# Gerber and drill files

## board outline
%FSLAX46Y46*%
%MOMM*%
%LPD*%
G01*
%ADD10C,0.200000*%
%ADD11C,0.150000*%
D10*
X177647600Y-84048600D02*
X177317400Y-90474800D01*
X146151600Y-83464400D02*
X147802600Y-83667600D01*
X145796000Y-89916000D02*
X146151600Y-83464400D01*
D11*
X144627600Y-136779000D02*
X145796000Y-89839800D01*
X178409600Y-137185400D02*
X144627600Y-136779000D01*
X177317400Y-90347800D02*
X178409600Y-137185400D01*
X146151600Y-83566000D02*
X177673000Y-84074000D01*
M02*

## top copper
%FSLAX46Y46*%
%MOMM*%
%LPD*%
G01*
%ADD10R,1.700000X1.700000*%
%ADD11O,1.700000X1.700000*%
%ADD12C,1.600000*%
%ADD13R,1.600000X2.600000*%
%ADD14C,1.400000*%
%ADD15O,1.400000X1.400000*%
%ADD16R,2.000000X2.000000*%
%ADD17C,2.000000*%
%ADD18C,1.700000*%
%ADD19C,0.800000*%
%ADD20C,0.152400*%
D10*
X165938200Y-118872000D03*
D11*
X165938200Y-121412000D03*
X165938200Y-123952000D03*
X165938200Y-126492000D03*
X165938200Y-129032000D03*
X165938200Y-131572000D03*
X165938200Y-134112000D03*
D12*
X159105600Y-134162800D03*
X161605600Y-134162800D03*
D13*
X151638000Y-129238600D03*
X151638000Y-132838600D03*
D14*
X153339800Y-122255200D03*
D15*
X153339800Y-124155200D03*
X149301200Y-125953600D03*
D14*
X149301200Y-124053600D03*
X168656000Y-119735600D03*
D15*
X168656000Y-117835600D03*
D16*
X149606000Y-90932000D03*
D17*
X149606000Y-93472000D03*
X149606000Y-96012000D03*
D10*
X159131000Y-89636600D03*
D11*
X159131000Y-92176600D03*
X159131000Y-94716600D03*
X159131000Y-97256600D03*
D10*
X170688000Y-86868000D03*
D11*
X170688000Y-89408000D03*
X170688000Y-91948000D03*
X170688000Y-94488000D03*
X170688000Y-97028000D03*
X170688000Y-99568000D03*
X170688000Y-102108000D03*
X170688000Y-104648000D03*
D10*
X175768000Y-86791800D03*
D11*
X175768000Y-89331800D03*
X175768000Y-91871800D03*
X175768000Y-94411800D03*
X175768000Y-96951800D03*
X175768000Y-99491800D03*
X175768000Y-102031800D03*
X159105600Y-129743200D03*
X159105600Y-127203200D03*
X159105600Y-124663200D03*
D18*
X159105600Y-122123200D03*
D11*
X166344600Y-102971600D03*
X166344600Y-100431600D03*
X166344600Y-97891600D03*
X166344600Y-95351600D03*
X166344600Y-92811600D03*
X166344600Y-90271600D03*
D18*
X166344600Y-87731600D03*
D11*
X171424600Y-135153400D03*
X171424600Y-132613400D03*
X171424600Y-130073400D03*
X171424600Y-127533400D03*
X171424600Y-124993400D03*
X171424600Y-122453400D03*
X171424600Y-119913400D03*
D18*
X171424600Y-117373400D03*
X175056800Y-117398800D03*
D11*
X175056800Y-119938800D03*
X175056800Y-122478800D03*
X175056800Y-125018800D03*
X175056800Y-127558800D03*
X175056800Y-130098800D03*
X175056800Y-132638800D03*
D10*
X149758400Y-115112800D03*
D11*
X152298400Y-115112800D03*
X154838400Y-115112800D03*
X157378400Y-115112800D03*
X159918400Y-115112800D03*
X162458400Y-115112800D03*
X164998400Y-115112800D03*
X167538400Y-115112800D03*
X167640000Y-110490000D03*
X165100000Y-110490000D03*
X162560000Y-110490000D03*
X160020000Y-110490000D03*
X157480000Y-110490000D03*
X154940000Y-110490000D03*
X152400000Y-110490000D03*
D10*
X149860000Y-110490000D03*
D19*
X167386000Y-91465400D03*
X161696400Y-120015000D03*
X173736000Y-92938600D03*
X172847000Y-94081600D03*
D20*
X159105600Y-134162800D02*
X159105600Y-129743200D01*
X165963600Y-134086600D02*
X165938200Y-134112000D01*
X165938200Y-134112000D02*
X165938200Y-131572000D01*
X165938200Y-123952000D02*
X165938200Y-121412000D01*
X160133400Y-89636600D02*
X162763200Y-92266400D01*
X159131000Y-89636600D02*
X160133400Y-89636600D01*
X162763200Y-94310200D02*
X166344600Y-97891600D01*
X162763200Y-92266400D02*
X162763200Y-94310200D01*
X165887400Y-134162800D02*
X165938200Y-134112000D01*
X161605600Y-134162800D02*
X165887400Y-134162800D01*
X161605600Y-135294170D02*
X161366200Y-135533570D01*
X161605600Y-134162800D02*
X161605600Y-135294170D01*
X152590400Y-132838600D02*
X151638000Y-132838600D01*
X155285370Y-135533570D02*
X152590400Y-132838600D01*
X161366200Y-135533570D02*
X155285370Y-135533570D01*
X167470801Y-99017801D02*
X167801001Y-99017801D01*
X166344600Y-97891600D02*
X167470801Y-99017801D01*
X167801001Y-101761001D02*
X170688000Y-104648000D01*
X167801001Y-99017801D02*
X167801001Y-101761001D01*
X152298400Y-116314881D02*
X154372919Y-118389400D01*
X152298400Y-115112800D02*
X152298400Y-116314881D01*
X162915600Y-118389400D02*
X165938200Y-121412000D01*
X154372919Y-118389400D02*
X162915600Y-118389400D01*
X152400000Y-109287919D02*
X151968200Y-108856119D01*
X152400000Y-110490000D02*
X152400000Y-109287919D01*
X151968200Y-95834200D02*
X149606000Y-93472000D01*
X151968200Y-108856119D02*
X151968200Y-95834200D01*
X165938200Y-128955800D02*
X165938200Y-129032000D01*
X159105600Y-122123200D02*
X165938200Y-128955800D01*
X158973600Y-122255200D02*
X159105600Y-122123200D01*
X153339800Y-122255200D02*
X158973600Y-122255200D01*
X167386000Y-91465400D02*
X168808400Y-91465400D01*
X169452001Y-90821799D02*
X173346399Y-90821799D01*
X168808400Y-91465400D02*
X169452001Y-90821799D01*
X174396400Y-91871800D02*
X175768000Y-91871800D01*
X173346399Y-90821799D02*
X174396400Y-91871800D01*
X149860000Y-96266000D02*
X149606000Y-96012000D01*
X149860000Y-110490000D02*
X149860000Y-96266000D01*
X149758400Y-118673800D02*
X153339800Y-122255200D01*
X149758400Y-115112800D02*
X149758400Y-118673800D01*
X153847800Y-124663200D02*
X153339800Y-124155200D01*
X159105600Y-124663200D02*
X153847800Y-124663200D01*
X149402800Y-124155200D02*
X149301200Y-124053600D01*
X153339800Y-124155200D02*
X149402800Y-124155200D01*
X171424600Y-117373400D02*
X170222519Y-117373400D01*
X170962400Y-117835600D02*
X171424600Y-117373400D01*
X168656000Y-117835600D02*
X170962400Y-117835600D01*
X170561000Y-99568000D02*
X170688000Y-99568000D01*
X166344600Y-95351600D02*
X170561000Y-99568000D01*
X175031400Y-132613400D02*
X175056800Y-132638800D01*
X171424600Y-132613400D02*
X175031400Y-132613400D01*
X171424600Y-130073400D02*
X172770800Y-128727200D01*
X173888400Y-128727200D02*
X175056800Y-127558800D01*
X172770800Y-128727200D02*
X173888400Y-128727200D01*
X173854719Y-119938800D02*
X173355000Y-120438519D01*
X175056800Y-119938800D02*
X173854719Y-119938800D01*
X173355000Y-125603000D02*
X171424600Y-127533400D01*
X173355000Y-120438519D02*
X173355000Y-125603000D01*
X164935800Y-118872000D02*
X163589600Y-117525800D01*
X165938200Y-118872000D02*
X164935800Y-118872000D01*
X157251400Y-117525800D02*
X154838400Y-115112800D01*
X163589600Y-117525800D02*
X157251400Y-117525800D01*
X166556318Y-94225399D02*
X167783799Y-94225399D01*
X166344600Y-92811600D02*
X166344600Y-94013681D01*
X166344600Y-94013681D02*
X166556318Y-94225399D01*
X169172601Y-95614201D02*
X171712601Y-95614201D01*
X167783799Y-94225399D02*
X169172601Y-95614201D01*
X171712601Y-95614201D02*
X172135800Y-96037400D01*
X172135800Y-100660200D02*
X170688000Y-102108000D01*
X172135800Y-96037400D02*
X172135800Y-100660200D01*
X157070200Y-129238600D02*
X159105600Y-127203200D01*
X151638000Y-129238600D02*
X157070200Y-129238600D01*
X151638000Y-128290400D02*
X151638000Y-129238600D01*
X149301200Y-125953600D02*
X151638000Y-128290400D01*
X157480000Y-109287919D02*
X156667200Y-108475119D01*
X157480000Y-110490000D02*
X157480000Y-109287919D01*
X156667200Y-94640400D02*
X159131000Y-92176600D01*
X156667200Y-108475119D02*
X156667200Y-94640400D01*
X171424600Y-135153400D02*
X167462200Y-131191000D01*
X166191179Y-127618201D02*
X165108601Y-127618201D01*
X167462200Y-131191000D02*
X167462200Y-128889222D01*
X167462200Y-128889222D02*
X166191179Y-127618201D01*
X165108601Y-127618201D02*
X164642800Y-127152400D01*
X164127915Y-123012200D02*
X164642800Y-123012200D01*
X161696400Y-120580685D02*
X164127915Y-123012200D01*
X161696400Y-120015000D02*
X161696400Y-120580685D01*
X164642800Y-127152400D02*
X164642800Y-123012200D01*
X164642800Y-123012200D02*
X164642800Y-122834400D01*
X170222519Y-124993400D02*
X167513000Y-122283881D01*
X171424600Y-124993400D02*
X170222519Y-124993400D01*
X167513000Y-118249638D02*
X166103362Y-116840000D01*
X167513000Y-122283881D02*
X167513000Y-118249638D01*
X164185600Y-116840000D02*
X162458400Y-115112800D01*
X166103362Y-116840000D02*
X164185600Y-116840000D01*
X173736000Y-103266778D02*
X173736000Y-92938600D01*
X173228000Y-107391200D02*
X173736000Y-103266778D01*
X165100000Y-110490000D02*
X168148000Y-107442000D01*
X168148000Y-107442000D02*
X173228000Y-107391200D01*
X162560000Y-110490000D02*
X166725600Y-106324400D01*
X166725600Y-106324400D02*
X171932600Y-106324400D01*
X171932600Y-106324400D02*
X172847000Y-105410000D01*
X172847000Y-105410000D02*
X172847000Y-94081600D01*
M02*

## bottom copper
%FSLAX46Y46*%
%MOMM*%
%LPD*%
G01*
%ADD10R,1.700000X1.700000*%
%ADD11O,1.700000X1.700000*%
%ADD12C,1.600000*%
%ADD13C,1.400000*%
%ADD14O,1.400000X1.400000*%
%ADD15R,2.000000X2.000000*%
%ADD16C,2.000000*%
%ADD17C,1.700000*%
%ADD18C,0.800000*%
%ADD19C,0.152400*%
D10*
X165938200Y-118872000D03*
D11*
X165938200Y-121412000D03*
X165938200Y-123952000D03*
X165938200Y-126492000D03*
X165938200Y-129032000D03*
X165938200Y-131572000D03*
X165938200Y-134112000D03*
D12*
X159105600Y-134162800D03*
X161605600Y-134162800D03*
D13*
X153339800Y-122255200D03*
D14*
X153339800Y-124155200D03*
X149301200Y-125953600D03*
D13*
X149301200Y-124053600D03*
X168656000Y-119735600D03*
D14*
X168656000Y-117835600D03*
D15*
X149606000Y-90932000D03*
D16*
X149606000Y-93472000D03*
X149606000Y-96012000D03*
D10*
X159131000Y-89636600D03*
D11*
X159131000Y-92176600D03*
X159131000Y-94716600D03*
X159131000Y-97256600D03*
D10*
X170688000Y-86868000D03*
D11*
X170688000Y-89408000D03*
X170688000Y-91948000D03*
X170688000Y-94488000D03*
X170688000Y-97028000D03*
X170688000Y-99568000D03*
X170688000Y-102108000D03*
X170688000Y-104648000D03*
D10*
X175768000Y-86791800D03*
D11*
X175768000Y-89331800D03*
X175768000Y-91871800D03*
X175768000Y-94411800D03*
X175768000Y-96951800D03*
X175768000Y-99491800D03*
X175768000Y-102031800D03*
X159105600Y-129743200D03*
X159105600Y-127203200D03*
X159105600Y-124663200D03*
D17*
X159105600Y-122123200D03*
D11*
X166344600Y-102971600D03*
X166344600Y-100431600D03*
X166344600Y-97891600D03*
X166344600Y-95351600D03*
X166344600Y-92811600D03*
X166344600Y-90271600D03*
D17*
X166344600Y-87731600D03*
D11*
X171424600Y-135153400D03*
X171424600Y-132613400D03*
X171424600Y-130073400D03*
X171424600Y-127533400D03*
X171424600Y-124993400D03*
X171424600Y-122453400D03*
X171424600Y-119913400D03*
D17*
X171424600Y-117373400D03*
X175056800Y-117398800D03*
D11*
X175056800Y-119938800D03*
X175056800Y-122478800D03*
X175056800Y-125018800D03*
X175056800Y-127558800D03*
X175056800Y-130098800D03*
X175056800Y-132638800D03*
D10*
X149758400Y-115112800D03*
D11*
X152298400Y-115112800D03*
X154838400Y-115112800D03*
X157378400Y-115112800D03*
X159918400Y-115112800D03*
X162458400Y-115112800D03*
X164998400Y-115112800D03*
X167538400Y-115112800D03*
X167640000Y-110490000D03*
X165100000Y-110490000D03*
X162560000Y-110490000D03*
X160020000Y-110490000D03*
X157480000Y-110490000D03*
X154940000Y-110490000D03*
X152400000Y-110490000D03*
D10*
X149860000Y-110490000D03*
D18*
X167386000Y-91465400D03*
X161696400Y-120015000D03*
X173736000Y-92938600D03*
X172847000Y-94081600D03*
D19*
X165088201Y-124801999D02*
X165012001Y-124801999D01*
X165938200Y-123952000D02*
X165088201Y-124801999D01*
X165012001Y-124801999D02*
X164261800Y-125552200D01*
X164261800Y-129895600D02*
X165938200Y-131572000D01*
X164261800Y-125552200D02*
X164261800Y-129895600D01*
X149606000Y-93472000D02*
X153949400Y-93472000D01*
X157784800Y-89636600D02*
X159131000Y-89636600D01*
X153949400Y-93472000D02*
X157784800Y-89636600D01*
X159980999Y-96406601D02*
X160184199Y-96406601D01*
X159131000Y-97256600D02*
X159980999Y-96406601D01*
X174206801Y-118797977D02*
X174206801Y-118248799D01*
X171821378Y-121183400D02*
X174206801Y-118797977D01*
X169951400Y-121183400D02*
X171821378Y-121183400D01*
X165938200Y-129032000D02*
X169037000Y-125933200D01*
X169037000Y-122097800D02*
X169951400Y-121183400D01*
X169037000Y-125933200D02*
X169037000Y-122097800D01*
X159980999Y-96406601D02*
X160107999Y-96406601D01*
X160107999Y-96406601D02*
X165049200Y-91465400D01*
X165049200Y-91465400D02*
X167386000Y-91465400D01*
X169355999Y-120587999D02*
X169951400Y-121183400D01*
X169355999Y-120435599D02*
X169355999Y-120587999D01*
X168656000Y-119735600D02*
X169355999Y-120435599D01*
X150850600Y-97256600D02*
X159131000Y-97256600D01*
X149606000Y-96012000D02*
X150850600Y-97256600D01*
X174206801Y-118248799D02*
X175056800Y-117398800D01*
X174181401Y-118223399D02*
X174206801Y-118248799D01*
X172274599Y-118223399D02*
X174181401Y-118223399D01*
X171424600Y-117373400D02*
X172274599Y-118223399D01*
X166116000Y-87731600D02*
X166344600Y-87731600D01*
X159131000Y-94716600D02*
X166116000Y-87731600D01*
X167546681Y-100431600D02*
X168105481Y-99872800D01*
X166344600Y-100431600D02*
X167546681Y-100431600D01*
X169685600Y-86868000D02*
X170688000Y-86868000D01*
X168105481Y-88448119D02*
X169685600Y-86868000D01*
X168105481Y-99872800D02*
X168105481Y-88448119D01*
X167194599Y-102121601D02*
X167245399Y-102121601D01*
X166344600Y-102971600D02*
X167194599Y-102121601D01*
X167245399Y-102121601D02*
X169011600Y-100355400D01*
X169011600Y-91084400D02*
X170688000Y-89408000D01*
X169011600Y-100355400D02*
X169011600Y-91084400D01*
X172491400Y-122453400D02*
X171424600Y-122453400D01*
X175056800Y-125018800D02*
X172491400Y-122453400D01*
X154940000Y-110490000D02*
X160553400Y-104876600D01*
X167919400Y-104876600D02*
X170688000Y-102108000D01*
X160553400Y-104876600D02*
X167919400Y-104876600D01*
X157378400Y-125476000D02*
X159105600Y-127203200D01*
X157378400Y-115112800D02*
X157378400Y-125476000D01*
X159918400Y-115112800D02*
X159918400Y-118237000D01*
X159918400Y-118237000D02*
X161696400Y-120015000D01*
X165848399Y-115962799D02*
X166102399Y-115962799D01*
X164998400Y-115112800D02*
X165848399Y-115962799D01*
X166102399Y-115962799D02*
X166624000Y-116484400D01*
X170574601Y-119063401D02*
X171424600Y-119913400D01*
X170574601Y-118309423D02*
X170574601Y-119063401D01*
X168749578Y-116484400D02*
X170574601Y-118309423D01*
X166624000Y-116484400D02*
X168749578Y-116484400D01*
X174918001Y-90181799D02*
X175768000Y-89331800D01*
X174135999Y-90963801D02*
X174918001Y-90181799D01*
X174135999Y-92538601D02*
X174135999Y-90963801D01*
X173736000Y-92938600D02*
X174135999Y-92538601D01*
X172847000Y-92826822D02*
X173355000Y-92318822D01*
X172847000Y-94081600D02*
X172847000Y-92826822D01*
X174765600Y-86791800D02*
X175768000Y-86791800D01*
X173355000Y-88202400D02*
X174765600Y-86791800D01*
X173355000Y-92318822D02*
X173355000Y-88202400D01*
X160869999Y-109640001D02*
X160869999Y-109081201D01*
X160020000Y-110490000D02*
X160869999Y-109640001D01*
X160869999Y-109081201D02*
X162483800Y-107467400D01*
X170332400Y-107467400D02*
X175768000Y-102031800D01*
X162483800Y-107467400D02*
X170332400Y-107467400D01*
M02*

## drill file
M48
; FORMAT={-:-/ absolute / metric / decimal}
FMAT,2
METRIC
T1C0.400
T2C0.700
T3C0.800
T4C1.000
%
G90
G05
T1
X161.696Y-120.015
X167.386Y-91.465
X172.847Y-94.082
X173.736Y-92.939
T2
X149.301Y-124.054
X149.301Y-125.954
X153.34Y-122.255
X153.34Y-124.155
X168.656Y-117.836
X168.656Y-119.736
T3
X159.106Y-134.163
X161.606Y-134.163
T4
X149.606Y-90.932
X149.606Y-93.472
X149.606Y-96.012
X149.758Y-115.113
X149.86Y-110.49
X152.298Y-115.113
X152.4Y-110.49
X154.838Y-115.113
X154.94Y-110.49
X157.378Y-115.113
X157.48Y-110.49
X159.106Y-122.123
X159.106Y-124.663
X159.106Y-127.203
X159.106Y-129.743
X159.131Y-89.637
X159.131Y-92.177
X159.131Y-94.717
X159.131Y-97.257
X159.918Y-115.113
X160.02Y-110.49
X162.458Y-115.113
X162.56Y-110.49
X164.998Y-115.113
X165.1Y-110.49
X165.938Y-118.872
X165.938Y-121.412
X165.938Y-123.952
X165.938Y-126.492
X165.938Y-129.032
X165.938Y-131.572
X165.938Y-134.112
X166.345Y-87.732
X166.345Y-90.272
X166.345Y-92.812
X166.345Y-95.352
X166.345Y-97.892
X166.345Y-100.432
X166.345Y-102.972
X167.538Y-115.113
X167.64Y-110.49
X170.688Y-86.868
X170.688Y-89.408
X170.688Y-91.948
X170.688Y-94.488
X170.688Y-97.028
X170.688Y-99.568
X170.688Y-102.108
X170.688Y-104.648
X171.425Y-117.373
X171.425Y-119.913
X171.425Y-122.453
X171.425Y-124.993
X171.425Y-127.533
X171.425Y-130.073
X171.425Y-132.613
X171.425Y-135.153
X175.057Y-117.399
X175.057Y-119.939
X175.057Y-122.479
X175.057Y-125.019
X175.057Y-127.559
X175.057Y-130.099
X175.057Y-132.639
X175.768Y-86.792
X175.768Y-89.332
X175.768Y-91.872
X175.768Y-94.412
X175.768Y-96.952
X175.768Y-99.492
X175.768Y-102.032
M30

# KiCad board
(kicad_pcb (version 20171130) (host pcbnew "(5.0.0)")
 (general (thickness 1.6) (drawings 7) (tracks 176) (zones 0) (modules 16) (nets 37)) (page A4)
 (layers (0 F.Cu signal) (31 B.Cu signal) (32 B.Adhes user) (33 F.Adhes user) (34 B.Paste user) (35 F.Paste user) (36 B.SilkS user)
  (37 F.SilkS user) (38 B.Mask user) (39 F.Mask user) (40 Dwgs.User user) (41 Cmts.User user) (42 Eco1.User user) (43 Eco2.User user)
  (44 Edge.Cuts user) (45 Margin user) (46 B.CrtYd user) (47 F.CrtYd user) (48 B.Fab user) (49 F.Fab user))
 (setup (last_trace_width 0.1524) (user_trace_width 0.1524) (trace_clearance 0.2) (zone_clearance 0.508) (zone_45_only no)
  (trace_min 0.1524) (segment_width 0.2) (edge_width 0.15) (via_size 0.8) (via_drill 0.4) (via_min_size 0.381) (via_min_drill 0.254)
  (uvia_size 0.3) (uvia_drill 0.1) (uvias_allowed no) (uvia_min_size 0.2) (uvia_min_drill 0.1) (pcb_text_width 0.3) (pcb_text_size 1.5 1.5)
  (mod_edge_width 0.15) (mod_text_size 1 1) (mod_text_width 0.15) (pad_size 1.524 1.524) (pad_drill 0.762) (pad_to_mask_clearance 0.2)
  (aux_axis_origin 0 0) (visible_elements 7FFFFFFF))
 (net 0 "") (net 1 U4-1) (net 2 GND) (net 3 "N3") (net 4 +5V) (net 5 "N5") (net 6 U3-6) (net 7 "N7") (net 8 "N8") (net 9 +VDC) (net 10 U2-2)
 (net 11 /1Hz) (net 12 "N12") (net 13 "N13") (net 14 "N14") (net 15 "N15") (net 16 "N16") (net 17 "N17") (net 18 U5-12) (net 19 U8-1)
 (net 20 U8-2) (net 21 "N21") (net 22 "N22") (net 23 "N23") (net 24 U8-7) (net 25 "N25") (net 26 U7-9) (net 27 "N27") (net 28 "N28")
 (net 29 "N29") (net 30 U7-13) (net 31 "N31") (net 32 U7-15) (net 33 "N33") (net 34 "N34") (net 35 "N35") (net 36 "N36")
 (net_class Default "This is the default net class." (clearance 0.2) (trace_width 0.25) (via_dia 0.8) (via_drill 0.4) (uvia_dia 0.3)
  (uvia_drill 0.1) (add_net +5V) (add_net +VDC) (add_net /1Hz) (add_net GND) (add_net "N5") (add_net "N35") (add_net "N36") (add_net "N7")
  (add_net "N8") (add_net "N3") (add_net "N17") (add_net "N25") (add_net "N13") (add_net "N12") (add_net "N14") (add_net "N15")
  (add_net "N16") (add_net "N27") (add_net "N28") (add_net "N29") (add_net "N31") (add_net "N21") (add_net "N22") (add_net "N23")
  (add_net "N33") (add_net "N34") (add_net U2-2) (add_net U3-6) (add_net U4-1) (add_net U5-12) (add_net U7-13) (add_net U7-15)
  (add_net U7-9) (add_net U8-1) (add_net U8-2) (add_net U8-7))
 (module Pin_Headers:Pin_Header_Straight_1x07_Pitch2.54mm (layer F.Cu) (at 165.9382 118.872)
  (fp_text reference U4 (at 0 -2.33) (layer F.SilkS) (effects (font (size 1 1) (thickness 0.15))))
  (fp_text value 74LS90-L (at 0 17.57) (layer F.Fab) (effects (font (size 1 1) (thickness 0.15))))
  (pad 1 thru_hole rect (at 0 0) (size 1.7 1.7) (drill 1) (layers *.Cu *.Mask) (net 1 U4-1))
  (pad 2 thru_hole oval (at 0 2.54) (size 1.7 1.7) (drill 1) (layers *.Cu *.Mask) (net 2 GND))
  (pad 3 thru_hole oval (at 0 5.08) (size 1.7 1.7) (drill 1) (layers *.Cu *.Mask) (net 2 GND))
  (pad 4 thru_hole oval (at 0 7.62) (size 1.7 1.7) (drill 1) (layers *.Cu *.Mask) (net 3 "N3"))
  (pad 5 thru_hole oval (at 0 10.16) (size 1.7 1.7) (drill 1) (layers *.Cu *.Mask) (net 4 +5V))
  (pad 6 thru_hole oval (at 0 12.7) (size 1.7 1.7) (drill 1) (layers *.Cu *.Mask) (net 2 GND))
  (pad 7 thru_hole oval (at 0 15.24) (size 1.7 1.7) (drill 1) (layers *.Cu *.Mask) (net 2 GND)))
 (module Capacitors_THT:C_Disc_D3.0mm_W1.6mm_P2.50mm (layer F.Cu) (at 159.1056 134.1628)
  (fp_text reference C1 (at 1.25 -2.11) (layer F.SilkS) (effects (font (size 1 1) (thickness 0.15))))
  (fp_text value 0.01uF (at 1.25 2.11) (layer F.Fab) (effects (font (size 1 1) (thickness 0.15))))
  (pad 1 thru_hole circle (at 0 0) (size 1.6 1.6) (drill 0.8) (layers *.Cu *.Mask) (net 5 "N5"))
  (pad 2 thru_hole circle (at 2.5 0) (size 1.6 1.6) (drill 0.8) (layers *.Cu *.Mask) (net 2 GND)))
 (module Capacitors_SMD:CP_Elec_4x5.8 (layer F.Cu) (at 151.638 131.0386 270)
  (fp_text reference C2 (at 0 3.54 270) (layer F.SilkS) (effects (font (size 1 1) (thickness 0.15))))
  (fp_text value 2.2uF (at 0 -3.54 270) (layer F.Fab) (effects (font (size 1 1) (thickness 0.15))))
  (pad 1 smd rect (at -1.8 0 90) (size 2.6 1.6) (layers F.Cu F.Paste F.Mask) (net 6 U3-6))
  (pad 2 smd rect (at 1.8 0 90) (size 2.6 1.6) (layers F.Cu F.Paste F.Mask) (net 2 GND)))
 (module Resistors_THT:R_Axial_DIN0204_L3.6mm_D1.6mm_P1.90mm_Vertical (layer F.Cu) (at 153.3398 122.2552 270)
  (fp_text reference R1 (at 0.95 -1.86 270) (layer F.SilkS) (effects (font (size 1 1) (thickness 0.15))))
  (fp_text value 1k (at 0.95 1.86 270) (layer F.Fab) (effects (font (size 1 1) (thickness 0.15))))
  (pad 1 thru_hole circle (at 0 0 270) (size 1.4 1.4) (drill 0.7) (layers *.Cu *.Mask) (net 4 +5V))
  (pad 2 thru_hole oval (at 1.9 0 270) (size 1.4 1.4) (drill 0.7) (layers *.Cu *.Mask) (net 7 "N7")))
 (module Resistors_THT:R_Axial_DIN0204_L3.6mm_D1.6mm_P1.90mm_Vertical (layer F.Cu) (at 149.3012 124.0536 270)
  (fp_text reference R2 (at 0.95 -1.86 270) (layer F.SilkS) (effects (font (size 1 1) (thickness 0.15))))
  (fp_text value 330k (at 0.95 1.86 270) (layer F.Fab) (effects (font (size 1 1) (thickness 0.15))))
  (pad 2 thru_hole oval (at 1.9 0 270) (size 1.4 1.4) (drill 0.7) (layers *.Cu *.Mask) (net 6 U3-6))
  (pad 1 thru_hole circle (at 0 0 270) (size 1.4 1.4) (drill 0.7) (layers *.Cu *.Mask) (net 7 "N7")))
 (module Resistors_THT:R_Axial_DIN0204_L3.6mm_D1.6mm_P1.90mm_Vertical (layer F.Cu) (at 168.656 119.7356 90)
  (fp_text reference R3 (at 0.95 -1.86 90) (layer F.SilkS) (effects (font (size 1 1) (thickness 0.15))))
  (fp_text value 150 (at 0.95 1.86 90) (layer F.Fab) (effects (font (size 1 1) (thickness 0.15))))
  (pad 1 thru_hole circle (at 0 0 90) (size 1.4 1.4) (drill 0.7) (layers *.Cu *.Mask) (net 4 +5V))
  (pad 2 thru_hole oval (at 1.9 0 90) (size 1.4 1.4) (drill 0.7) (layers *.Cu *.Mask) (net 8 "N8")))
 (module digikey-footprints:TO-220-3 (layer F.Cu) (at 149.606 90.932 270)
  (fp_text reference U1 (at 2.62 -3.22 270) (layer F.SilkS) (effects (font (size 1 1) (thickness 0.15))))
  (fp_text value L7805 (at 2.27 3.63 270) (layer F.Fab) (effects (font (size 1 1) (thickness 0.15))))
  (pad 1 thru_hole rect (at 0 0 270) (size 2 2) (drill 1) (layers *.Cu *.Mask) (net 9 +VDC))
  (pad 2 thru_hole circle (at 2.54 0 270) (size 2 2) (drill 1) (layers *.Cu *.Mask) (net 2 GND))
  (pad 3 thru_hole circle (at 5.08 0 270) (size 2 2) (drill 1) (layers *.Cu *.Mask) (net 4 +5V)))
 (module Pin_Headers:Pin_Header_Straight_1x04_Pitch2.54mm (layer F.Cu) (at 159.131 89.6366)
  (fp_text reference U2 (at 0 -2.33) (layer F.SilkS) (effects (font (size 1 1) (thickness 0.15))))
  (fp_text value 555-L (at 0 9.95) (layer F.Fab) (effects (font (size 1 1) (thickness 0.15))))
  (pad 1 thru_hole rect (at 0 0) (size 1.7 1.7) (drill 1) (layers *.Cu *.Mask) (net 2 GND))
  (pad 2 thru_hole oval (at 0 2.54) (size 1.7 1.7) (drill 1) (layers *.Cu *.Mask) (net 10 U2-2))
  (pad 3 thru_hole oval (at 0 5.08) (size 1.7 1.7) (drill 1) (layers *.Cu *.Mask) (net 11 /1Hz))
  (pad 4 thru_hole oval (at 0 7.62) (size 1.7 1.7) (drill 1) (layers *.Cu *.Mask) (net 4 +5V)))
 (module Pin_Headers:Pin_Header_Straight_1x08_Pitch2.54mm (layer F.Cu) (at 170.688 86.868)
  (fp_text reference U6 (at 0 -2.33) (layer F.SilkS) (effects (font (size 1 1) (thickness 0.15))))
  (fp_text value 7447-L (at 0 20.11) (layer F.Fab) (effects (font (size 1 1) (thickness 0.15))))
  (pad 1 thru_hole rect (at 0 0) (size 1.7 1.7) (drill 1) (layers *.Cu *.Mask) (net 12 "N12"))
  (pad 2 thru_hole oval (at 0 2.54) (size 1.7 1.7) (drill 1) (layers *.Cu *.Mask) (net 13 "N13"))
  (pad 3 thru_hole oval (at 0 5.08) (size 1.7 1.7) (drill 1) (layers *.Cu *.Mask) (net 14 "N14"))
  (pad 4 thru_hole oval (at 0 7.62) (size 1.7 1.7) (drill 1) (layers *.Cu *.Mask) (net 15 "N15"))
  (pad 5 thru_hole oval (at 0 10.16) (size 1.7 1.7) (drill 1) (layers *.Cu *.Mask) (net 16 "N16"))
  (pad 6 thru_hole oval (at 0 12.7) (size 1.7 1.7) (drill 1) (layers *.Cu *.Mask) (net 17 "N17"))
  (pad 7 thru_hole oval (at 0 15.24) (size 1.7 1.7) (drill 1) (layers *.Cu *.Mask) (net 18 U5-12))
  (pad 8 thru_hole oval (at 0 17.78) (size 1.7 1.7) (drill 1) (layers *.Cu *.Mask) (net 2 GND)))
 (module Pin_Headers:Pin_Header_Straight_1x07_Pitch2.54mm (layer F.Cu) (at 175.768 86.7918)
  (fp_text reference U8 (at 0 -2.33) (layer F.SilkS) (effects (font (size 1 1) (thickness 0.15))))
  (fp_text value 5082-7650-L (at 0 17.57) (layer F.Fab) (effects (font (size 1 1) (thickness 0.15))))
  (pad 1 thru_hole rect (at 0 0) (size 1.7 1.7) (drill 1) (layers *.Cu *.Mask) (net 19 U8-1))
  (pad 2 thru_hole oval (at 0 2.54) (size 1.7 1.7) (drill 1) (layers *.Cu *.Mask) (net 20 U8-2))
  (pad 3 thru_hole oval (at 0 5.08) (size 1.7 1.7) (drill 1) (layers *.Cu *.Mask) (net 4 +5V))
  (pad 4 thru_hole oval (at 0 7.62) (size 1.7 1.7) (drill 1) (layers *.Cu *.Mask) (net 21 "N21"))
  (pad 5 thru_hole oval (at 0 10.16) (size 1.7 1.7) (drill 1) (layers *.Cu *.Mask) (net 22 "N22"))
  (pad 6 thru_hole oval (at 0 12.7) (size 1.7 1.7) (drill 1) (layers *.Cu *.Mask) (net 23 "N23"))
  (pad 7 thru_hole oval (at 0 15.24) (size 1.7 1.7) (drill 1) (layers *.Cu *.Mask) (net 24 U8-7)))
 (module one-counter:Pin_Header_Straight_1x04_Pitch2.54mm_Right (layer F.Cu) (at 159.1056 122.1232)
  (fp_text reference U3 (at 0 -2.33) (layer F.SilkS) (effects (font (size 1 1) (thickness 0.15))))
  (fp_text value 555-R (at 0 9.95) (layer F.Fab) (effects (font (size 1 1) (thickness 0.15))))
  (pad 5 thru_hole oval (at 0 7.62) (size 1.7 1.7) (drill 1) (layers *.Cu *.Mask) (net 5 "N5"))
  (pad 6 thru_hole oval (at 0 5.08) (size 1.7 1.7) (drill 1) (layers *.Cu *.Mask) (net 6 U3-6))
  (pad 7 thru_hole oval (at 0 2.54) (size 1.7 1.7) (drill 1) (layers *.Cu *.Mask) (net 7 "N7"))
  (pad 8 thru_hole circle (at 0 0) (size 1.7 1.7) (drill 1) (layers *.Cu *.Mask) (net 4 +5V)))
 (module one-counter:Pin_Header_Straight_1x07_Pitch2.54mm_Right (layer F.Cu) (at 166.3446 87.7316)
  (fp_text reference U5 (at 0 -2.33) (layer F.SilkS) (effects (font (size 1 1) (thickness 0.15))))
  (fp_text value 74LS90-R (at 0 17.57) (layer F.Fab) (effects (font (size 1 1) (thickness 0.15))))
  (pad 8 thru_hole oval (at 0 15.24) (size 1.7 1.7) (drill 1) (layers *.Cu *.Mask) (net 13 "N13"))
  (pad 9 thru_hole oval (at 0 12.7) (size 1.7 1.7) (drill 1) (layers *.Cu *.Mask) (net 12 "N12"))
  (pad 10 thru_hole oval (at 0 10.16) (size 1.7 1.7) (drill 1) (layers *.Cu *.Mask) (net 2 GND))
  (pad 11 thru_hole oval (at 0 7.62) (size 1.7 1.7) (drill 1) (layers *.Cu *.Mask) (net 17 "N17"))
  (pad 12 thru_hole oval (at 0 5.08) (size 1.7 1.7) (drill 1) (layers *.Cu *.Mask) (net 18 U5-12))
  (pad 13 thru_hole oval (at 0 2.54) (size 1.7 1.7) (drill 1) (layers *.Cu *.Mask) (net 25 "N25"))
  (pad 14 thru_hole circle (at 0 0) (size 1.7 1.7) (drill 1) (layers *.Cu *.Mask) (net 11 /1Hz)))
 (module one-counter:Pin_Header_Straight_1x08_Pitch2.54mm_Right (layer F.Cu) (at 171.4246 117.3734)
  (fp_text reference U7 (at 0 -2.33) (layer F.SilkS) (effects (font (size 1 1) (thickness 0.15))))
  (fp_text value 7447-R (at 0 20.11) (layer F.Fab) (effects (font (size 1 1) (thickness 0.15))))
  (pad 9 thru_hole oval (at 0 17.78) (size 1.7 1.7) (drill 1) (layers *.Cu *.Mask) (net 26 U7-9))
  (pad 10 thru_hole oval (at 0 15.24) (size 1.7 1.7) (drill 1) (layers *.Cu *.Mask) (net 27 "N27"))
  (pad 11 thru_hole oval (at 0 12.7) (size 1.7 1.7) (drill 1) (layers *.Cu *.Mask) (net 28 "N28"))
  (pad 12 thru_hole oval (at 0 10.16) (size 1.7 1.7) (drill 1) (layers *.Cu *.Mask) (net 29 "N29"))
  (pad 13 thru_hole oval (at 0 7.62) (size 1.7 1.7) (drill 1) (layers *.Cu *.Mask) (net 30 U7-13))
  (pad 14 thru_hole oval (at 0 5.08) (size 1.7 1.7) (drill 1) (layers *.Cu *.Mask) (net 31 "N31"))
  (pad 15 thru_hole oval (at 0 2.54) (size 1.7 1.7) (drill 1) (layers *.Cu *.Mask) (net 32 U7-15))
  (pad 16 thru_hole circle (at 0 0) (size 1.7 1.7) (drill 1) (layers *.Cu *.Mask) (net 4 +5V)))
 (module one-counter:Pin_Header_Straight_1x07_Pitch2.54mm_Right (layer F.Cu) (at 175.0568 117.3988)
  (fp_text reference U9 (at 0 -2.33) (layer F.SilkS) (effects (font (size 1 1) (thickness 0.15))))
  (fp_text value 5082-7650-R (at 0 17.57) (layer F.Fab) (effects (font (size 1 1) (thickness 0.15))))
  (pad 14 thru_hole circle (at 0 0) (size 1.7 1.7) (drill 1) (layers *.Cu *.Mask) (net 4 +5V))
  (pad 13 thru_hole oval (at 0 2.54) (size 1.7 1.7) (drill 1) (layers *.Cu *.Mask) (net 29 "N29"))
  (pad 12 thru_hole oval (at 0 5.08) (size 1.7 1.7) (drill 1) (layers *.Cu *.Mask) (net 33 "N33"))
  (pad 11 thru_hole oval (at 0 7.62) (size 1.7 1.7) (drill 1) (layers *.Cu *.Mask) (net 31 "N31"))
  (pad 10 thru_hole oval (at 0 10.16) (size 1.7 1.7) (drill 1) (layers *.Cu *.Mask) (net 28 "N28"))
  (pad 9 thru_hole oval (at 0 12.7) (size 1.7 1.7) (drill 1) (layers *.Cu *.Mask) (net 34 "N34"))
  (pad 8 thru_hole oval (at 0 15.24) (size 1.7 1.7) (drill 1) (layers *.Cu *.Mask) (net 27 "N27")))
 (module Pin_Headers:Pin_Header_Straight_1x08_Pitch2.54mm (layer F.Cu) (at 149.7584 115.1128 90)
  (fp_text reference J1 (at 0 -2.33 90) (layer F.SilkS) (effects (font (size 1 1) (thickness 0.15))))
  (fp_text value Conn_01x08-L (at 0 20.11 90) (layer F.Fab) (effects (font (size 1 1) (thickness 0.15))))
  (pad 1 thru_hole rect (at 0 0 90) (size 1.7 1.7) (drill 1) (layers *.Cu *.Mask) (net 4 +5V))
  (pad 2 thru_hole oval (at 0 2.54 90) (size 1.7 1.7) (drill 1) (layers *.Cu *.Mask) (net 2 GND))
  (pad 3 thru_hole oval (at 0 5.08 90) (size 1.7 1.7) (drill 1) (layers *.Cu *.Mask) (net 1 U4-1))
  (pad 4 thru_hole oval (at 0 7.62 90) (size 1.7 1.7) (drill 1) (layers *.Cu *.Mask) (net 6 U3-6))
  (pad 5 thru_hole oval (at 0 10.16 90) (size 1.7 1.7) (drill 1) (layers *.Cu *.Mask) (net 26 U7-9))
  (pad 6 thru_hole oval (at 0 12.7 90) (size 1.7 1.7) (drill 1) (layers *.Cu *.Mask) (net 30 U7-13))
  (pad 7 thru_hole oval (at 0 15.24 90) (size 1.7 1.7) (drill 1) (layers *.Cu *.Mask) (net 32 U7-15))
  (pad 8 thru_hole oval (at 0 17.78 90) (size 1.7 1.7) (drill 1) (layers *.Cu *.Mask) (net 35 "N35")))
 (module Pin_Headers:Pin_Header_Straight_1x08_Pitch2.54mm (layer F.Cu) (at 149.86 110.49 90)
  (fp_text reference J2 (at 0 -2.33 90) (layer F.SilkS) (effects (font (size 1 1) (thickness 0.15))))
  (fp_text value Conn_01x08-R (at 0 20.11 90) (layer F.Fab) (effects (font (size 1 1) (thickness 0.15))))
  (pad 8 thru_hole oval (at 0 17.78 90) (size 1.7 1.7) (drill 1) (layers *.Cu *.Mask) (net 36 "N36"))
  (pad 7 thru_hole oval (at 0 15.24 90) (size 1.7 1.7) (drill 1) (layers *.Cu *.Mask) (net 20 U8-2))
  (pad 6 thru_hole oval (at 0 12.7 90) (size 1.7 1.7) (drill 1) (layers *.Cu *.Mask) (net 19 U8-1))
  (pad 5 thru_hole oval (at 0 10.16 90) (size 1.7 1.7) (drill 1) (layers *.Cu *.Mask) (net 24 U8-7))
  (pad 4 thru_hole oval (at 0 7.62 90) (size 1.7 1.7) (drill 1) (layers *.Cu *.Mask) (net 10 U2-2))
  (pad 3 thru_hole oval (at 0 5.08 90) (size 1.7 1.7) (drill 1) (layers *.Cu *.Mask) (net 18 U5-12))
  (pad 2 thru_hole oval (at 0 2.54 90) (size 1.7 1.7) (drill 1) (layers *.Cu *.Mask) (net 2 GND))
  (pad 1 thru_hole rect (at 0 0 90) (size 1.7 1.7) (drill 1) (layers *.Cu *.Mask) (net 4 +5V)))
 (gr_line (start 177.6476 84.0486) (end 177.3174 90.4748) (layer Edge.Cuts) (width 0.2))
 (gr_line (start 146.1516 83.4644) (end 147.8026 83.6676) (layer Edge.Cuts) (width 0.2))
 (gr_line (start 145.796 89.916) (end 146.1516 83.4644) (layer Edge.Cuts) (width 0.2))
 (gr_line (start 144.6276 136.779) (end 145.796 89.8398) (layer Edge.Cuts) (width 0.15))
 (gr_line (start 178.4096 137.1854) (end 144.6276 136.779) (layer Edge.Cuts) (width 0.15))
 (gr_line (start 177.3174 90.3478) (end 178.4096 137.1854) (layer Edge.Cuts) (width 0.15))
 (gr_line (start 146.1516 83.566) (end 177.673 84.074) (layer Edge.Cuts) (width 0.15))
 (segment (start 159.1056 134.1628) (end 159.1056 129.7432) (width 0.1524) (layer F.Cu) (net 5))
 (segment (start 165.9636 134.0866) (end 165.9382 134.112) (width 0.1524) (layer F.Cu) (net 2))
 (segment (start 165.9382 134.112) (end 165.9382 131.572) (width 0.1524) (layer F.Cu) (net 2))
 (segment (start 165.9382 123.952) (end 165.9382 121.412) (width 0.1524) (layer F.Cu) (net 2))
 (segment (start 160.1334 89.6366) (end 162.7632 92.2664) (width 0.1524) (layer F.Cu) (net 2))
 (segment (start 159.131 89.6366) (end 160.1334 89.6366) (width 0.1524) (layer F.Cu) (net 2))
 (segment (start 162.7632 94.3102) (end 166.3446 97.8916) (width 0.1524) (layer F.Cu) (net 2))
 (segment (start 162.7632 92.2664) (end 162.7632 94.3102) (width 0.1524) (layer F.Cu) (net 2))
 (segment (start 165.8874 134.1628) (end 165.9382 134.112) (width 0.1524) (layer F.Cu) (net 2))
 (segment (start 161.6056 134.1628) (end 165.8874 134.1628) (width 0.1524) (layer F.Cu) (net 2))
 (segment (start 161.6056 135.29417) (end 161.3662 135.53357) (width 0.1524) (layer F.Cu) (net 2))
 (segment (start 161.6056 134.1628) (end 161.6056 135.29417) (width 0.1524) (layer F.Cu) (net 2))
 (segment (start 152.5904 132.8386) (end 151.638 132.8386) (width 0.1524) (layer F.Cu) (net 2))
 (segment (start 155.28537 135.53357) (end 152.5904 132.8386) (width 0.1524) (layer F.Cu) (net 2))
 (segment (start 161.3662 135.53357) (end 155.28537 135.53357) (width 0.1524) (layer F.Cu) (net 2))
 (segment (start 165.088201 124.801999) (end 165.012001 124.801999) (width 0.1524) (layer B.Cu) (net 2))
 (segment (start 165.9382 123.952) (end 165.088201 124.801999) (width 0.1524) (layer B.Cu) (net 2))
 (segment (start 165.012001 124.801999) (end 164.2618 125.5522) (width 0.1524) (layer B.Cu) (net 2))
 (segment (start 164.2618 129.8956) (end 165.9382 131.572) (width 0.1524) (layer B.Cu) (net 2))
 (segment (start 164.2618 125.5522) (end 164.2618 129.8956) (width 0.1524) (layer B.Cu) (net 2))
 (segment (start 149.606 93.472) (end 153.9494 93.472) (width 0.1524) (layer B.Cu) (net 2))
 (segment (start 157.7848 89.6366) (end 159.131 89.6366) (width 0.1524) (layer B.Cu) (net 2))
 (segment (start 153.9494 93.472) (end 157.7848 89.6366) (width 0.1524) (layer B.Cu) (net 2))
 (segment (start 167.470801 99.017801) (end 167.801001 99.017801) (width 0.1524) (layer F.Cu) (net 2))
 (segment (start 166.3446 97.8916) (end 167.470801 99.017801) (width 0.1524) (layer F.Cu) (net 2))
 (segment (start 167.801001 101.761001) (end 170.688 104.648) (width 0.1524) (layer F.Cu) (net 2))
 (segment (start 167.801001 99.017801) (end 167.801001 101.761001) (width 0.1524) (layer F.Cu) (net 2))
 (segment (start 152.2984 116.314881) (end 154.372919 118.3894) (width 0.1524) (layer F.Cu) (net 2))
 (segment (start 152.2984 115.1128) (end 152.2984 116.314881) (width 0.1524) (layer F.Cu) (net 2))
 (segment (start 162.9156 118.3894) (end 165.9382 121.412) (width 0.1524) (layer F.Cu) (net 2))
 (segment (start 154.372919 118.3894) (end 162.9156 118.3894) (width 0.1524) (layer F.Cu) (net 2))
 (segment (start 152.4 109.287919) (end 151.9682 108.856119) (width 0.1524) (layer F.Cu) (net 2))
 (segment (start 152.4 110.49) (end 152.4 109.287919) (width 0.1524) (layer F.Cu) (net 2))
 (segment (start 151.9682 95.8342) (end 149.606 93.472) (width 0.1524) (layer F.Cu) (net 2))
 (segment (start 151.9682 108.856119) (end 151.9682 95.8342) (width 0.1524) (layer F.Cu) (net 2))
 (segment (start 159.980999 96.406601) (end 160.184199 96.406601) (width 0.1524) (layer B.Cu) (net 4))
 (segment (start 159.131 97.2566) (end 159.980999 96.406601) (width 0.1524) (layer B.Cu) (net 4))
 (segment (start 174.206801 118.797977) (end 174.206801 118.248799) (width 0.1524) (layer B.Cu) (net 4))
 (segment (start 171.821378 121.1834) (end 174.206801 118.797977) (width 0.1524) (layer B.Cu) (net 4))
 (segment (start 169.9514 121.1834) (end 171.821378 121.1834) (width 0.1524) (layer B.Cu) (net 4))
 (segment (start 165.9382 128.9558) (end 165.9382 129.032) (width 0.1524) (layer F.Cu) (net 4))
 (segment (start 159.1056 122.1232) (end 165.9382 128.9558) (width 0.1524) (layer F.Cu) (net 4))
 (segment (start 158.9736 122.2552) (end 159.1056 122.1232) (width 0.1524) (layer F.Cu) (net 4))
 (segment (start 153.3398 122.2552) (end 158.9736 122.2552) (width 0.1524) (layer F.Cu) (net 4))
 (segment (start 165.9382 129.032) (end 169.037 125.9332) (width 0.1524) (layer B.Cu) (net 4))
 (segment (start 169.037 122.0978) (end 169.9514 121.1834) (width 0.1524) (layer B.Cu) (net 4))
 (segment (start 169.037 125.9332) (end 169.037 122.0978) (width 0.1524) (layer B.Cu) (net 4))
 (segment (start 159.980999 96.406601) (end 160.107999 96.406601) (width 0.1524) (layer B.Cu) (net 4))
 (via (at 167.386 91.4654) (size 0.8) (drill 0.4) (layers F.Cu B.Cu) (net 4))
 (segment (start 160.107999 96.406601) (end 165.0492 91.4654) (width 0.1524) (layer B.Cu) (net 4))
 (segment (start 165.0492 91.4654) (end 167.386 91.4654) (width 0.1524) (layer B.Cu) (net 4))
 (segment (start 167.386 91.4654) (end 168.8084 91.4654) (width 0.1524) (layer F.Cu) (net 4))
 (segment (start 169.452001 90.821799) (end 173.346399 90.821799) (width 0.1524) (layer F.Cu) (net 4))
 (segment (start 168.8084 91.4654) (end 169.452001 90.821799) (width 0.1524) (layer F.Cu) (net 4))
 (segment (start 174.3964 91.8718) (end 175.768 91.8718) (width 0.1524) (layer F.Cu) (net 4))
 (segment (start 173.346399 90.821799) (end 174.3964 91.8718) (width 0.1524) (layer F.Cu) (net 4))
 (segment (start 149.86 96.266) (end 149.606 96.012) (width 0.1524) (layer F.Cu) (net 4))
 (segment (start 149.86 110.49) (end 149.86 96.266) (width 0.1524) (layer F.Cu) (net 4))
 (segment (start 149.7584 118.6738) (end 153.3398 122.2552) (width 0.1524) (layer F.Cu) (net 4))
 (segment (start 149.7584 115.1128) (end 149.7584 118.6738) (width 0.1524) (layer F.Cu) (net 4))
 (segment (start 169.355999 120.587999) (end 169.9514 121.1834) (width 0.1524) (layer B.Cu) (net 4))
 (segment (start 169.355999 120.435599) (end 169.355999 120.587999) (width 0.1524) (layer B.Cu) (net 4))
 (segment (start 168.656 119.7356) (end 169.355999 120.435599) (width 0.1524) (layer B.Cu) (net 4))
 (segment (start 150.8506 97.2566) (end 159.131 97.2566) (width 0.1524) (layer B.Cu) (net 4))
 (segment (start 149.606 96.012) (end 150.8506 97.2566) (width 0.1524) (layer B.Cu) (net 4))
 (segment (start 174.206801 118.248799) (end 175.0568 117.3988) (width 0.1524) (layer B.Cu) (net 4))
 (segment (start 174.181401 118.223399) (end 174.206801 118.248799) (width 0.1524) (layer B.Cu) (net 4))
 (segment (start 172.274599 118.223399) (end 174.181401 118.223399) (width 0.1524) (layer B.Cu) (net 4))
 (segment (start 171.4246 117.3734) (end 172.274599 118.223399) (width 0.1524) (layer B.Cu) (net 4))
 (segment (start 153.8478 124.6632) (end 153.3398 124.1552) (width 0.1524) (layer F.Cu) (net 7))
 (segment (start 159.1056 124.6632) (end 153.8478 124.6632) (width 0.1524) (layer F.Cu) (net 7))
 (segment (start 149.4028 124.1552) (end 149.3012 124.0536) (width 0.1524) (layer F.Cu) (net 7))
 (segment (start 153.3398 124.1552) (end 149.4028 124.1552) (width 0.1524) (layer F.Cu) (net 7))
 (segment (start 171.4246 117.3734) (end 170.222519 117.3734) (width 0.1524) (layer F.Cu) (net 8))
 (segment (start 170.9624 117.8356) (end 171.4246 117.3734) (width 0.1524) (layer F.Cu) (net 8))
 (segment (start 168.656 117.8356) (end 170.9624 117.8356) (width 0.1524) (layer F.Cu) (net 8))
 (segment (start 166.116 87.7316) (end 166.3446 87.7316) (width 0.1524) (layer B.Cu) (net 11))
 (segment (start 159.131 94.7166) (end 166.116 87.7316) (width 0.1524) (layer B.Cu) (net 11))
 (segment (start 167.546681 100.4316) (end 168.105481 99.8728) (width 0.1524) (layer B.Cu) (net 12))
 (segment (start 166.3446 100.4316) (end 167.546681 100.4316) (width 0.1524) (layer B.Cu) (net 12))
 (segment (start 169.6856 86.868) (end 170.688 86.868) (width 0.1524) (layer B.Cu) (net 12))
 (segment (start 168.105481 88.448119) (end 169.6856 86.868) (width 0.1524) (layer B.Cu) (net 12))
 (segment (start 168.105481 99.8728) (end 168.105481 88.448119) (width 0.1524) (layer B.Cu) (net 12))
 (segment (start 167.194599 102.121601) (end 167.245399 102.121601) (width 0.1524) (layer B.Cu) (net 13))
 (segment (start 166.3446 102.9716) (end 167.194599 102.121601) (width 0.1524) (layer B.Cu) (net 13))
 (segment (start 167.245399 102.121601) (end 169.0116 100.3554) (width 0.1524) (layer B.Cu) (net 13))
 (segment (start 169.0116 91.0844) (end 170.688 89.408) (width 0.1524) (layer B.Cu) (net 13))
 (segment (start 169.0116 100.3554) (end 169.0116 91.0844) (width 0.1524) (layer B.Cu) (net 13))
 (segment (start 170.561 99.568) (end 170.688 99.568) (width 0.1524) (layer F.Cu) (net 17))
 (segment (start 166.3446 95.3516) (end 170.561 99.568) (width 0.1524) (layer F.Cu) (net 17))
 (segment (start 175.0314 132.6134) (end 175.0568 132.6388) (width 0.1524) (layer F.Cu) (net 27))
 (segment (start 171.4246 132.6134) (end 175.0314 132.6134) (width 0.1524) (layer F.Cu) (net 27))
 (segment (start 171.4246 130.0734) (end 172.7708 128.7272) (width 0.1524) (layer F.Cu) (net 28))
 (segment (start 173.8884 128.7272) (end 175.0568 127.5588) (width 0.1524) (layer F.Cu) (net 28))
 (segment (start 172.7708 128.7272) (end 173.8884 128.7272) (width 0.1524) (layer F.Cu) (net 28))
 (segment (start 173.854719 119.9388) (end 173.355 120.438519) (width 0.1524) (layer F.Cu) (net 29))
 (segment (start 175.0568 119.9388) (end 173.854719 119.9388) (width 0.1524) (layer F.Cu) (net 29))
 (segment (start 173.355 125.603) (end 171.4246 127.5334) (width 0.1524) (layer F.Cu) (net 29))
 (segment (start 173.355 120.438519) (end 173.355 125.603) (width 0.1524) (layer F.Cu) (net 29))
 (segment (start 172.4914 122.4534) (end 171.4246 122.4534) (width 0.1524) (layer B.Cu) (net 31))
 (segment (start 175.0568 125.0188) (end 172.4914 122.4534) (width 0.1524) (layer B.Cu) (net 31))
 (segment (start 164.9358 118.872) (end 163.5896 117.5258) (width 0.1524) (layer F.Cu) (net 1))
 (segment (start 165.9382 118.872) (end 164.9358 118.872) (width 0.1524) (layer F.Cu) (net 1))
 (segment (start 157.2514 117.5258) (end 154.8384 115.1128) (width 0.1524) (layer F.Cu) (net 1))
 (segment (start 163.5896 117.5258) (end 157.2514 117.5258) (width 0.1524) (layer F.Cu) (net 1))
 (segment (start 166.556318 94.225399) (end 167.783799 94.225399) (width 0.1524) (layer F.Cu) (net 18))
 (segment (start 166.3446 92.8116) (end 166.3446 94.013681) (width 0.1524) (layer F.Cu) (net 18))
 (segment (start 166.3446 94.013681) (end 166.556318 94.225399) (width 0.1524) (layer F.Cu) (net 18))
 (segment (start 169.172601 95.614201) (end 171.712601 95.614201) (width 0.1524) (layer F.Cu) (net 18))
 (segment (start 167.783799 94.225399) (end 169.172601 95.614201) (width 0.1524) (layer F.Cu) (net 18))
 (segment (start 171.712601 95.614201) (end 172.1358 96.0374) (width 0.1524) (layer F.Cu) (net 18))
 (segment (start 172.1358 100.6602) (end 170.688 102.108) (width 0.1524) (layer F.Cu) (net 18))
 (segment (start 172.1358 96.0374) (end 172.1358 100.6602) (width 0.1524) (layer F.Cu) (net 18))
 (segment (start 154.94 110.49) (end 160.5534 104.8766) (width 0.1524) (layer B.Cu) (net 18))
 (segment (start 167.9194 104.8766) (end 170.688 102.108) (width 0.1524) (layer B.Cu) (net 18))
 (segment (start 160.5534 104.8766) (end 167.9194 104.8766) (width 0.1524) (layer B.Cu) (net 18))
 (segment (start 157.0702 129.2386) (end 159.1056 127.2032) (width 0.1524) (layer F.Cu) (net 6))
 (segment (start 151.638 129.2386) (end 157.0702 129.2386) (width 0.1524) (layer F.Cu) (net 6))
 (segment (start 151.638 128.2904) (end 151.638 129.2386) (width 0.1524) (layer F.Cu) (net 6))
 (segment (start 149.3012 125.9536) (end 151.638 128.2904) (width 0.1524) (layer F.Cu) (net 6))
 (segment (start 157.3784 125.476) (end 159.1056 127.2032) (width 0.1524) (layer B.Cu) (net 6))
 (segment (start 157.3784 115.1128) (end 157.3784 125.476) (width 0.1524) (layer B.Cu) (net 6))
 (segment (start 157.48 109.287919) (end 156.6672 108.475119) (width 0.1524) (layer F.Cu) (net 10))
 (segment (start 157.48 110.49) (end 157.48 109.287919) (width 0.1524) (layer F.Cu) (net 10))
 (segment (start 156.6672 94.6404) (end 159.131 92.1766) (width 0.1524) (layer F.Cu) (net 10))
 (segment (start 156.6672 108.475119) (end 156.6672 94.6404) (width 0.1524) (layer F.Cu) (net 10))
 (segment (start 171.4246 135.1534) (end 167.4622 131.191) (width 0.1524) (layer F.Cu) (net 26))
 (segment (start 166.191179 127.618201) (end 165.108601 127.618201) (width 0.1524) (layer F.Cu) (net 26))
 (segment (start 167.4622 131.191) (end 167.4622 128.889222) (width 0.1524) (layer F.Cu) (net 26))
 (segment (start 167.4622 128.889222) (end 166.191179 127.618201) (width 0.1524) (layer F.Cu) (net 26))
 (segment (start 165.108601 127.618201) (end 164.6428 127.1524) (width 0.1524) (layer F.Cu) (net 26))
 (via (at 161.6964 120.015) (size 0.8) (drill 0.4) (layers F.Cu B.Cu) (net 26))
 (segment (start 159.9184 115.1128) (end 159.9184 118.237) (width 0.1524) (layer B.Cu) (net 26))
 (segment (start 159.9184 118.237) (end 161.6964 120.015) (width 0.1524) (layer B.Cu) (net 26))
 (segment (start 164.127915 123.0122) (end 164.6428 123.0122) (width 0.1524) (layer F.Cu) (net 26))
 (segment (start 161.6964 120.580685) (end 164.127915 123.0122) (width 0.1524) (layer F.Cu) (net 26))
 (segment (start 161.6964 120.015) (end 161.6964 120.580685) (width 0.1524) (layer F.Cu) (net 26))
 (segment (start 164.6428 127.1524) (end 164.6428 123.0122) (width 0.1524) (layer F.Cu) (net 26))
 (segment (start 164.6428 123.0122) (end 164.6428 122.8344) (width 0.1524) (layer F.Cu) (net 26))
 (segment (start 170.222519 124.9934) (end 167.513 122.283881) (width 0.1524) (layer F.Cu) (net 30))
 (segment (start 171.4246 124.9934) (end 170.222519 124.9934) (width 0.1524) (layer F.Cu) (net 30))
 (segment (start 167.513 118.249638) (end 166.103362 116.84) (width 0.1524) (layer F.Cu) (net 30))
 (segment (start 167.513 122.283881) (end 167.513 118.249638) (width 0.1524) (layer F.Cu) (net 30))
 (segment (start 164.1856 116.84) (end 162.4584 115.1128) (width 0.1524) (layer F.Cu) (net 30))
 (segment (start 166.103362 116.84) (end 164.1856 116.84) (width 0.1524) (layer F.Cu) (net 30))
 (segment (start 165.848399 115.962799) (end 166.102399 115.962799) (width 0.1524) (layer B.Cu) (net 32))
 (segment (start 164.9984 115.1128) (end 165.848399 115.962799) (width 0.1524) (layer B.Cu) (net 32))
 (segment (start 166.102399 115.962799) (end 166.624 116.4844) (width 0.1524) (layer B.Cu) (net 32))
 (segment (start 170.574601 119.063401) (end 171.4246 119.9134) (width 0.1524) (layer B.Cu) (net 32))
 (segment (start 170.574601 118.309423) (end 170.574601 119.063401) (width 0.1524) (layer B.Cu) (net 32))
 (segment (start 168.749578 116.4844) (end 170.574601 118.309423) (width 0.1524) (layer B.Cu) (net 32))
 (segment (start 166.624 116.4844) (end 168.749578 116.4844) (width 0.1524) (layer B.Cu) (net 32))
 (via (at 173.736 92.9386) (size 0.8) (drill 0.4) (layers F.Cu B.Cu) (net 20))
 (segment (start 174.918001 90.181799) (end 175.768 89.3318) (width 0.1524) (layer B.Cu) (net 20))
 (segment (start 174.135999 90.963801) (end 174.918001 90.181799) (width 0.1524) (layer B.Cu) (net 20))
 (segment (start 174.135999 92.538601) (end 174.135999 90.963801) (width 0.1524) (layer B.Cu) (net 20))
 (segment (start 173.736 92.9386) (end 174.135999 92.538601) (width 0.1524) (layer B.Cu) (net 20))
 (segment (start 173.736 103.266778) (end 173.736 92.9386) (width 0.1524) (layer F.Cu) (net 20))
 (segment (start 173.228 107.3912) (end 173.736 103.266778) (width 0.1524) (layer F.Cu) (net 20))
 (segment (start 165.1 110.49) (end 168.148 107.442) (width 0.1524) (layer F.Cu) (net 20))
 (segment (start 168.148 107.442) (end 173.228 107.3912) (width 0.1524) (layer F.Cu) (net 20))
 (segment (start 162.56 110.49) (end 166.7256 106.3244) (width 0.1524) (layer F.Cu) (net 19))
 (segment (start 166.7256 106.3244) (end 171.9326 106.3244) (width 0.1524) (layer F.Cu) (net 19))
 (via (at 172.847 94.0816) (size 0.8) (drill 0.4) (layers F.Cu B.Cu) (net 19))
 (segment (start 171.9326 106.3244) (end 172.847 105.41) (width 0.1524) (layer F.Cu) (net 19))
 (segment (start 172.847 105.41) (end 172.847 94.0816) (width 0.1524) (layer F.Cu) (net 19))
 (segment (start 172.847 92.826822) (end 173.355 92.318822) (width 0.1524) (layer B.Cu) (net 19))
 (segment (start 172.847 94.0816) (end 172.847 92.826822) (width 0.1524) (layer B.Cu) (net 19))
 (segment (start 174.7656 86.7918) (end 175.768 86.7918) (width 0.1524) (layer B.Cu) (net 19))
 (segment (start 173.355 88.2024) (end 174.7656 86.7918) (width 0.1524) (layer B.Cu) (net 19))
 (segment (start 173.355 92.318822) (end 173.355 88.2024) (width 0.1524) (layer B.Cu) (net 19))
 (segment (start 160.869999 109.640001) (end 160.869999 109.081201) (width 0.1524) (layer B.Cu) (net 24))
 (segment (start 160.02 110.49) (end 160.869999 109.640001) (width 0.1524) (layer B.Cu) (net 24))
 (segment (start 160.869999 109.081201) (end 162.4838 107.4674) (width 0.1524) (layer B.Cu) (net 24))
 (segment (start 170.3324 107.4674) (end 175.768 102.0318) (width 0.1524) (layer B.Cu) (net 24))
 (segment (start 162.4838 107.4674) (end 170.3324 107.4674) (width 0.1524) (layer B.Cu) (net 24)))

